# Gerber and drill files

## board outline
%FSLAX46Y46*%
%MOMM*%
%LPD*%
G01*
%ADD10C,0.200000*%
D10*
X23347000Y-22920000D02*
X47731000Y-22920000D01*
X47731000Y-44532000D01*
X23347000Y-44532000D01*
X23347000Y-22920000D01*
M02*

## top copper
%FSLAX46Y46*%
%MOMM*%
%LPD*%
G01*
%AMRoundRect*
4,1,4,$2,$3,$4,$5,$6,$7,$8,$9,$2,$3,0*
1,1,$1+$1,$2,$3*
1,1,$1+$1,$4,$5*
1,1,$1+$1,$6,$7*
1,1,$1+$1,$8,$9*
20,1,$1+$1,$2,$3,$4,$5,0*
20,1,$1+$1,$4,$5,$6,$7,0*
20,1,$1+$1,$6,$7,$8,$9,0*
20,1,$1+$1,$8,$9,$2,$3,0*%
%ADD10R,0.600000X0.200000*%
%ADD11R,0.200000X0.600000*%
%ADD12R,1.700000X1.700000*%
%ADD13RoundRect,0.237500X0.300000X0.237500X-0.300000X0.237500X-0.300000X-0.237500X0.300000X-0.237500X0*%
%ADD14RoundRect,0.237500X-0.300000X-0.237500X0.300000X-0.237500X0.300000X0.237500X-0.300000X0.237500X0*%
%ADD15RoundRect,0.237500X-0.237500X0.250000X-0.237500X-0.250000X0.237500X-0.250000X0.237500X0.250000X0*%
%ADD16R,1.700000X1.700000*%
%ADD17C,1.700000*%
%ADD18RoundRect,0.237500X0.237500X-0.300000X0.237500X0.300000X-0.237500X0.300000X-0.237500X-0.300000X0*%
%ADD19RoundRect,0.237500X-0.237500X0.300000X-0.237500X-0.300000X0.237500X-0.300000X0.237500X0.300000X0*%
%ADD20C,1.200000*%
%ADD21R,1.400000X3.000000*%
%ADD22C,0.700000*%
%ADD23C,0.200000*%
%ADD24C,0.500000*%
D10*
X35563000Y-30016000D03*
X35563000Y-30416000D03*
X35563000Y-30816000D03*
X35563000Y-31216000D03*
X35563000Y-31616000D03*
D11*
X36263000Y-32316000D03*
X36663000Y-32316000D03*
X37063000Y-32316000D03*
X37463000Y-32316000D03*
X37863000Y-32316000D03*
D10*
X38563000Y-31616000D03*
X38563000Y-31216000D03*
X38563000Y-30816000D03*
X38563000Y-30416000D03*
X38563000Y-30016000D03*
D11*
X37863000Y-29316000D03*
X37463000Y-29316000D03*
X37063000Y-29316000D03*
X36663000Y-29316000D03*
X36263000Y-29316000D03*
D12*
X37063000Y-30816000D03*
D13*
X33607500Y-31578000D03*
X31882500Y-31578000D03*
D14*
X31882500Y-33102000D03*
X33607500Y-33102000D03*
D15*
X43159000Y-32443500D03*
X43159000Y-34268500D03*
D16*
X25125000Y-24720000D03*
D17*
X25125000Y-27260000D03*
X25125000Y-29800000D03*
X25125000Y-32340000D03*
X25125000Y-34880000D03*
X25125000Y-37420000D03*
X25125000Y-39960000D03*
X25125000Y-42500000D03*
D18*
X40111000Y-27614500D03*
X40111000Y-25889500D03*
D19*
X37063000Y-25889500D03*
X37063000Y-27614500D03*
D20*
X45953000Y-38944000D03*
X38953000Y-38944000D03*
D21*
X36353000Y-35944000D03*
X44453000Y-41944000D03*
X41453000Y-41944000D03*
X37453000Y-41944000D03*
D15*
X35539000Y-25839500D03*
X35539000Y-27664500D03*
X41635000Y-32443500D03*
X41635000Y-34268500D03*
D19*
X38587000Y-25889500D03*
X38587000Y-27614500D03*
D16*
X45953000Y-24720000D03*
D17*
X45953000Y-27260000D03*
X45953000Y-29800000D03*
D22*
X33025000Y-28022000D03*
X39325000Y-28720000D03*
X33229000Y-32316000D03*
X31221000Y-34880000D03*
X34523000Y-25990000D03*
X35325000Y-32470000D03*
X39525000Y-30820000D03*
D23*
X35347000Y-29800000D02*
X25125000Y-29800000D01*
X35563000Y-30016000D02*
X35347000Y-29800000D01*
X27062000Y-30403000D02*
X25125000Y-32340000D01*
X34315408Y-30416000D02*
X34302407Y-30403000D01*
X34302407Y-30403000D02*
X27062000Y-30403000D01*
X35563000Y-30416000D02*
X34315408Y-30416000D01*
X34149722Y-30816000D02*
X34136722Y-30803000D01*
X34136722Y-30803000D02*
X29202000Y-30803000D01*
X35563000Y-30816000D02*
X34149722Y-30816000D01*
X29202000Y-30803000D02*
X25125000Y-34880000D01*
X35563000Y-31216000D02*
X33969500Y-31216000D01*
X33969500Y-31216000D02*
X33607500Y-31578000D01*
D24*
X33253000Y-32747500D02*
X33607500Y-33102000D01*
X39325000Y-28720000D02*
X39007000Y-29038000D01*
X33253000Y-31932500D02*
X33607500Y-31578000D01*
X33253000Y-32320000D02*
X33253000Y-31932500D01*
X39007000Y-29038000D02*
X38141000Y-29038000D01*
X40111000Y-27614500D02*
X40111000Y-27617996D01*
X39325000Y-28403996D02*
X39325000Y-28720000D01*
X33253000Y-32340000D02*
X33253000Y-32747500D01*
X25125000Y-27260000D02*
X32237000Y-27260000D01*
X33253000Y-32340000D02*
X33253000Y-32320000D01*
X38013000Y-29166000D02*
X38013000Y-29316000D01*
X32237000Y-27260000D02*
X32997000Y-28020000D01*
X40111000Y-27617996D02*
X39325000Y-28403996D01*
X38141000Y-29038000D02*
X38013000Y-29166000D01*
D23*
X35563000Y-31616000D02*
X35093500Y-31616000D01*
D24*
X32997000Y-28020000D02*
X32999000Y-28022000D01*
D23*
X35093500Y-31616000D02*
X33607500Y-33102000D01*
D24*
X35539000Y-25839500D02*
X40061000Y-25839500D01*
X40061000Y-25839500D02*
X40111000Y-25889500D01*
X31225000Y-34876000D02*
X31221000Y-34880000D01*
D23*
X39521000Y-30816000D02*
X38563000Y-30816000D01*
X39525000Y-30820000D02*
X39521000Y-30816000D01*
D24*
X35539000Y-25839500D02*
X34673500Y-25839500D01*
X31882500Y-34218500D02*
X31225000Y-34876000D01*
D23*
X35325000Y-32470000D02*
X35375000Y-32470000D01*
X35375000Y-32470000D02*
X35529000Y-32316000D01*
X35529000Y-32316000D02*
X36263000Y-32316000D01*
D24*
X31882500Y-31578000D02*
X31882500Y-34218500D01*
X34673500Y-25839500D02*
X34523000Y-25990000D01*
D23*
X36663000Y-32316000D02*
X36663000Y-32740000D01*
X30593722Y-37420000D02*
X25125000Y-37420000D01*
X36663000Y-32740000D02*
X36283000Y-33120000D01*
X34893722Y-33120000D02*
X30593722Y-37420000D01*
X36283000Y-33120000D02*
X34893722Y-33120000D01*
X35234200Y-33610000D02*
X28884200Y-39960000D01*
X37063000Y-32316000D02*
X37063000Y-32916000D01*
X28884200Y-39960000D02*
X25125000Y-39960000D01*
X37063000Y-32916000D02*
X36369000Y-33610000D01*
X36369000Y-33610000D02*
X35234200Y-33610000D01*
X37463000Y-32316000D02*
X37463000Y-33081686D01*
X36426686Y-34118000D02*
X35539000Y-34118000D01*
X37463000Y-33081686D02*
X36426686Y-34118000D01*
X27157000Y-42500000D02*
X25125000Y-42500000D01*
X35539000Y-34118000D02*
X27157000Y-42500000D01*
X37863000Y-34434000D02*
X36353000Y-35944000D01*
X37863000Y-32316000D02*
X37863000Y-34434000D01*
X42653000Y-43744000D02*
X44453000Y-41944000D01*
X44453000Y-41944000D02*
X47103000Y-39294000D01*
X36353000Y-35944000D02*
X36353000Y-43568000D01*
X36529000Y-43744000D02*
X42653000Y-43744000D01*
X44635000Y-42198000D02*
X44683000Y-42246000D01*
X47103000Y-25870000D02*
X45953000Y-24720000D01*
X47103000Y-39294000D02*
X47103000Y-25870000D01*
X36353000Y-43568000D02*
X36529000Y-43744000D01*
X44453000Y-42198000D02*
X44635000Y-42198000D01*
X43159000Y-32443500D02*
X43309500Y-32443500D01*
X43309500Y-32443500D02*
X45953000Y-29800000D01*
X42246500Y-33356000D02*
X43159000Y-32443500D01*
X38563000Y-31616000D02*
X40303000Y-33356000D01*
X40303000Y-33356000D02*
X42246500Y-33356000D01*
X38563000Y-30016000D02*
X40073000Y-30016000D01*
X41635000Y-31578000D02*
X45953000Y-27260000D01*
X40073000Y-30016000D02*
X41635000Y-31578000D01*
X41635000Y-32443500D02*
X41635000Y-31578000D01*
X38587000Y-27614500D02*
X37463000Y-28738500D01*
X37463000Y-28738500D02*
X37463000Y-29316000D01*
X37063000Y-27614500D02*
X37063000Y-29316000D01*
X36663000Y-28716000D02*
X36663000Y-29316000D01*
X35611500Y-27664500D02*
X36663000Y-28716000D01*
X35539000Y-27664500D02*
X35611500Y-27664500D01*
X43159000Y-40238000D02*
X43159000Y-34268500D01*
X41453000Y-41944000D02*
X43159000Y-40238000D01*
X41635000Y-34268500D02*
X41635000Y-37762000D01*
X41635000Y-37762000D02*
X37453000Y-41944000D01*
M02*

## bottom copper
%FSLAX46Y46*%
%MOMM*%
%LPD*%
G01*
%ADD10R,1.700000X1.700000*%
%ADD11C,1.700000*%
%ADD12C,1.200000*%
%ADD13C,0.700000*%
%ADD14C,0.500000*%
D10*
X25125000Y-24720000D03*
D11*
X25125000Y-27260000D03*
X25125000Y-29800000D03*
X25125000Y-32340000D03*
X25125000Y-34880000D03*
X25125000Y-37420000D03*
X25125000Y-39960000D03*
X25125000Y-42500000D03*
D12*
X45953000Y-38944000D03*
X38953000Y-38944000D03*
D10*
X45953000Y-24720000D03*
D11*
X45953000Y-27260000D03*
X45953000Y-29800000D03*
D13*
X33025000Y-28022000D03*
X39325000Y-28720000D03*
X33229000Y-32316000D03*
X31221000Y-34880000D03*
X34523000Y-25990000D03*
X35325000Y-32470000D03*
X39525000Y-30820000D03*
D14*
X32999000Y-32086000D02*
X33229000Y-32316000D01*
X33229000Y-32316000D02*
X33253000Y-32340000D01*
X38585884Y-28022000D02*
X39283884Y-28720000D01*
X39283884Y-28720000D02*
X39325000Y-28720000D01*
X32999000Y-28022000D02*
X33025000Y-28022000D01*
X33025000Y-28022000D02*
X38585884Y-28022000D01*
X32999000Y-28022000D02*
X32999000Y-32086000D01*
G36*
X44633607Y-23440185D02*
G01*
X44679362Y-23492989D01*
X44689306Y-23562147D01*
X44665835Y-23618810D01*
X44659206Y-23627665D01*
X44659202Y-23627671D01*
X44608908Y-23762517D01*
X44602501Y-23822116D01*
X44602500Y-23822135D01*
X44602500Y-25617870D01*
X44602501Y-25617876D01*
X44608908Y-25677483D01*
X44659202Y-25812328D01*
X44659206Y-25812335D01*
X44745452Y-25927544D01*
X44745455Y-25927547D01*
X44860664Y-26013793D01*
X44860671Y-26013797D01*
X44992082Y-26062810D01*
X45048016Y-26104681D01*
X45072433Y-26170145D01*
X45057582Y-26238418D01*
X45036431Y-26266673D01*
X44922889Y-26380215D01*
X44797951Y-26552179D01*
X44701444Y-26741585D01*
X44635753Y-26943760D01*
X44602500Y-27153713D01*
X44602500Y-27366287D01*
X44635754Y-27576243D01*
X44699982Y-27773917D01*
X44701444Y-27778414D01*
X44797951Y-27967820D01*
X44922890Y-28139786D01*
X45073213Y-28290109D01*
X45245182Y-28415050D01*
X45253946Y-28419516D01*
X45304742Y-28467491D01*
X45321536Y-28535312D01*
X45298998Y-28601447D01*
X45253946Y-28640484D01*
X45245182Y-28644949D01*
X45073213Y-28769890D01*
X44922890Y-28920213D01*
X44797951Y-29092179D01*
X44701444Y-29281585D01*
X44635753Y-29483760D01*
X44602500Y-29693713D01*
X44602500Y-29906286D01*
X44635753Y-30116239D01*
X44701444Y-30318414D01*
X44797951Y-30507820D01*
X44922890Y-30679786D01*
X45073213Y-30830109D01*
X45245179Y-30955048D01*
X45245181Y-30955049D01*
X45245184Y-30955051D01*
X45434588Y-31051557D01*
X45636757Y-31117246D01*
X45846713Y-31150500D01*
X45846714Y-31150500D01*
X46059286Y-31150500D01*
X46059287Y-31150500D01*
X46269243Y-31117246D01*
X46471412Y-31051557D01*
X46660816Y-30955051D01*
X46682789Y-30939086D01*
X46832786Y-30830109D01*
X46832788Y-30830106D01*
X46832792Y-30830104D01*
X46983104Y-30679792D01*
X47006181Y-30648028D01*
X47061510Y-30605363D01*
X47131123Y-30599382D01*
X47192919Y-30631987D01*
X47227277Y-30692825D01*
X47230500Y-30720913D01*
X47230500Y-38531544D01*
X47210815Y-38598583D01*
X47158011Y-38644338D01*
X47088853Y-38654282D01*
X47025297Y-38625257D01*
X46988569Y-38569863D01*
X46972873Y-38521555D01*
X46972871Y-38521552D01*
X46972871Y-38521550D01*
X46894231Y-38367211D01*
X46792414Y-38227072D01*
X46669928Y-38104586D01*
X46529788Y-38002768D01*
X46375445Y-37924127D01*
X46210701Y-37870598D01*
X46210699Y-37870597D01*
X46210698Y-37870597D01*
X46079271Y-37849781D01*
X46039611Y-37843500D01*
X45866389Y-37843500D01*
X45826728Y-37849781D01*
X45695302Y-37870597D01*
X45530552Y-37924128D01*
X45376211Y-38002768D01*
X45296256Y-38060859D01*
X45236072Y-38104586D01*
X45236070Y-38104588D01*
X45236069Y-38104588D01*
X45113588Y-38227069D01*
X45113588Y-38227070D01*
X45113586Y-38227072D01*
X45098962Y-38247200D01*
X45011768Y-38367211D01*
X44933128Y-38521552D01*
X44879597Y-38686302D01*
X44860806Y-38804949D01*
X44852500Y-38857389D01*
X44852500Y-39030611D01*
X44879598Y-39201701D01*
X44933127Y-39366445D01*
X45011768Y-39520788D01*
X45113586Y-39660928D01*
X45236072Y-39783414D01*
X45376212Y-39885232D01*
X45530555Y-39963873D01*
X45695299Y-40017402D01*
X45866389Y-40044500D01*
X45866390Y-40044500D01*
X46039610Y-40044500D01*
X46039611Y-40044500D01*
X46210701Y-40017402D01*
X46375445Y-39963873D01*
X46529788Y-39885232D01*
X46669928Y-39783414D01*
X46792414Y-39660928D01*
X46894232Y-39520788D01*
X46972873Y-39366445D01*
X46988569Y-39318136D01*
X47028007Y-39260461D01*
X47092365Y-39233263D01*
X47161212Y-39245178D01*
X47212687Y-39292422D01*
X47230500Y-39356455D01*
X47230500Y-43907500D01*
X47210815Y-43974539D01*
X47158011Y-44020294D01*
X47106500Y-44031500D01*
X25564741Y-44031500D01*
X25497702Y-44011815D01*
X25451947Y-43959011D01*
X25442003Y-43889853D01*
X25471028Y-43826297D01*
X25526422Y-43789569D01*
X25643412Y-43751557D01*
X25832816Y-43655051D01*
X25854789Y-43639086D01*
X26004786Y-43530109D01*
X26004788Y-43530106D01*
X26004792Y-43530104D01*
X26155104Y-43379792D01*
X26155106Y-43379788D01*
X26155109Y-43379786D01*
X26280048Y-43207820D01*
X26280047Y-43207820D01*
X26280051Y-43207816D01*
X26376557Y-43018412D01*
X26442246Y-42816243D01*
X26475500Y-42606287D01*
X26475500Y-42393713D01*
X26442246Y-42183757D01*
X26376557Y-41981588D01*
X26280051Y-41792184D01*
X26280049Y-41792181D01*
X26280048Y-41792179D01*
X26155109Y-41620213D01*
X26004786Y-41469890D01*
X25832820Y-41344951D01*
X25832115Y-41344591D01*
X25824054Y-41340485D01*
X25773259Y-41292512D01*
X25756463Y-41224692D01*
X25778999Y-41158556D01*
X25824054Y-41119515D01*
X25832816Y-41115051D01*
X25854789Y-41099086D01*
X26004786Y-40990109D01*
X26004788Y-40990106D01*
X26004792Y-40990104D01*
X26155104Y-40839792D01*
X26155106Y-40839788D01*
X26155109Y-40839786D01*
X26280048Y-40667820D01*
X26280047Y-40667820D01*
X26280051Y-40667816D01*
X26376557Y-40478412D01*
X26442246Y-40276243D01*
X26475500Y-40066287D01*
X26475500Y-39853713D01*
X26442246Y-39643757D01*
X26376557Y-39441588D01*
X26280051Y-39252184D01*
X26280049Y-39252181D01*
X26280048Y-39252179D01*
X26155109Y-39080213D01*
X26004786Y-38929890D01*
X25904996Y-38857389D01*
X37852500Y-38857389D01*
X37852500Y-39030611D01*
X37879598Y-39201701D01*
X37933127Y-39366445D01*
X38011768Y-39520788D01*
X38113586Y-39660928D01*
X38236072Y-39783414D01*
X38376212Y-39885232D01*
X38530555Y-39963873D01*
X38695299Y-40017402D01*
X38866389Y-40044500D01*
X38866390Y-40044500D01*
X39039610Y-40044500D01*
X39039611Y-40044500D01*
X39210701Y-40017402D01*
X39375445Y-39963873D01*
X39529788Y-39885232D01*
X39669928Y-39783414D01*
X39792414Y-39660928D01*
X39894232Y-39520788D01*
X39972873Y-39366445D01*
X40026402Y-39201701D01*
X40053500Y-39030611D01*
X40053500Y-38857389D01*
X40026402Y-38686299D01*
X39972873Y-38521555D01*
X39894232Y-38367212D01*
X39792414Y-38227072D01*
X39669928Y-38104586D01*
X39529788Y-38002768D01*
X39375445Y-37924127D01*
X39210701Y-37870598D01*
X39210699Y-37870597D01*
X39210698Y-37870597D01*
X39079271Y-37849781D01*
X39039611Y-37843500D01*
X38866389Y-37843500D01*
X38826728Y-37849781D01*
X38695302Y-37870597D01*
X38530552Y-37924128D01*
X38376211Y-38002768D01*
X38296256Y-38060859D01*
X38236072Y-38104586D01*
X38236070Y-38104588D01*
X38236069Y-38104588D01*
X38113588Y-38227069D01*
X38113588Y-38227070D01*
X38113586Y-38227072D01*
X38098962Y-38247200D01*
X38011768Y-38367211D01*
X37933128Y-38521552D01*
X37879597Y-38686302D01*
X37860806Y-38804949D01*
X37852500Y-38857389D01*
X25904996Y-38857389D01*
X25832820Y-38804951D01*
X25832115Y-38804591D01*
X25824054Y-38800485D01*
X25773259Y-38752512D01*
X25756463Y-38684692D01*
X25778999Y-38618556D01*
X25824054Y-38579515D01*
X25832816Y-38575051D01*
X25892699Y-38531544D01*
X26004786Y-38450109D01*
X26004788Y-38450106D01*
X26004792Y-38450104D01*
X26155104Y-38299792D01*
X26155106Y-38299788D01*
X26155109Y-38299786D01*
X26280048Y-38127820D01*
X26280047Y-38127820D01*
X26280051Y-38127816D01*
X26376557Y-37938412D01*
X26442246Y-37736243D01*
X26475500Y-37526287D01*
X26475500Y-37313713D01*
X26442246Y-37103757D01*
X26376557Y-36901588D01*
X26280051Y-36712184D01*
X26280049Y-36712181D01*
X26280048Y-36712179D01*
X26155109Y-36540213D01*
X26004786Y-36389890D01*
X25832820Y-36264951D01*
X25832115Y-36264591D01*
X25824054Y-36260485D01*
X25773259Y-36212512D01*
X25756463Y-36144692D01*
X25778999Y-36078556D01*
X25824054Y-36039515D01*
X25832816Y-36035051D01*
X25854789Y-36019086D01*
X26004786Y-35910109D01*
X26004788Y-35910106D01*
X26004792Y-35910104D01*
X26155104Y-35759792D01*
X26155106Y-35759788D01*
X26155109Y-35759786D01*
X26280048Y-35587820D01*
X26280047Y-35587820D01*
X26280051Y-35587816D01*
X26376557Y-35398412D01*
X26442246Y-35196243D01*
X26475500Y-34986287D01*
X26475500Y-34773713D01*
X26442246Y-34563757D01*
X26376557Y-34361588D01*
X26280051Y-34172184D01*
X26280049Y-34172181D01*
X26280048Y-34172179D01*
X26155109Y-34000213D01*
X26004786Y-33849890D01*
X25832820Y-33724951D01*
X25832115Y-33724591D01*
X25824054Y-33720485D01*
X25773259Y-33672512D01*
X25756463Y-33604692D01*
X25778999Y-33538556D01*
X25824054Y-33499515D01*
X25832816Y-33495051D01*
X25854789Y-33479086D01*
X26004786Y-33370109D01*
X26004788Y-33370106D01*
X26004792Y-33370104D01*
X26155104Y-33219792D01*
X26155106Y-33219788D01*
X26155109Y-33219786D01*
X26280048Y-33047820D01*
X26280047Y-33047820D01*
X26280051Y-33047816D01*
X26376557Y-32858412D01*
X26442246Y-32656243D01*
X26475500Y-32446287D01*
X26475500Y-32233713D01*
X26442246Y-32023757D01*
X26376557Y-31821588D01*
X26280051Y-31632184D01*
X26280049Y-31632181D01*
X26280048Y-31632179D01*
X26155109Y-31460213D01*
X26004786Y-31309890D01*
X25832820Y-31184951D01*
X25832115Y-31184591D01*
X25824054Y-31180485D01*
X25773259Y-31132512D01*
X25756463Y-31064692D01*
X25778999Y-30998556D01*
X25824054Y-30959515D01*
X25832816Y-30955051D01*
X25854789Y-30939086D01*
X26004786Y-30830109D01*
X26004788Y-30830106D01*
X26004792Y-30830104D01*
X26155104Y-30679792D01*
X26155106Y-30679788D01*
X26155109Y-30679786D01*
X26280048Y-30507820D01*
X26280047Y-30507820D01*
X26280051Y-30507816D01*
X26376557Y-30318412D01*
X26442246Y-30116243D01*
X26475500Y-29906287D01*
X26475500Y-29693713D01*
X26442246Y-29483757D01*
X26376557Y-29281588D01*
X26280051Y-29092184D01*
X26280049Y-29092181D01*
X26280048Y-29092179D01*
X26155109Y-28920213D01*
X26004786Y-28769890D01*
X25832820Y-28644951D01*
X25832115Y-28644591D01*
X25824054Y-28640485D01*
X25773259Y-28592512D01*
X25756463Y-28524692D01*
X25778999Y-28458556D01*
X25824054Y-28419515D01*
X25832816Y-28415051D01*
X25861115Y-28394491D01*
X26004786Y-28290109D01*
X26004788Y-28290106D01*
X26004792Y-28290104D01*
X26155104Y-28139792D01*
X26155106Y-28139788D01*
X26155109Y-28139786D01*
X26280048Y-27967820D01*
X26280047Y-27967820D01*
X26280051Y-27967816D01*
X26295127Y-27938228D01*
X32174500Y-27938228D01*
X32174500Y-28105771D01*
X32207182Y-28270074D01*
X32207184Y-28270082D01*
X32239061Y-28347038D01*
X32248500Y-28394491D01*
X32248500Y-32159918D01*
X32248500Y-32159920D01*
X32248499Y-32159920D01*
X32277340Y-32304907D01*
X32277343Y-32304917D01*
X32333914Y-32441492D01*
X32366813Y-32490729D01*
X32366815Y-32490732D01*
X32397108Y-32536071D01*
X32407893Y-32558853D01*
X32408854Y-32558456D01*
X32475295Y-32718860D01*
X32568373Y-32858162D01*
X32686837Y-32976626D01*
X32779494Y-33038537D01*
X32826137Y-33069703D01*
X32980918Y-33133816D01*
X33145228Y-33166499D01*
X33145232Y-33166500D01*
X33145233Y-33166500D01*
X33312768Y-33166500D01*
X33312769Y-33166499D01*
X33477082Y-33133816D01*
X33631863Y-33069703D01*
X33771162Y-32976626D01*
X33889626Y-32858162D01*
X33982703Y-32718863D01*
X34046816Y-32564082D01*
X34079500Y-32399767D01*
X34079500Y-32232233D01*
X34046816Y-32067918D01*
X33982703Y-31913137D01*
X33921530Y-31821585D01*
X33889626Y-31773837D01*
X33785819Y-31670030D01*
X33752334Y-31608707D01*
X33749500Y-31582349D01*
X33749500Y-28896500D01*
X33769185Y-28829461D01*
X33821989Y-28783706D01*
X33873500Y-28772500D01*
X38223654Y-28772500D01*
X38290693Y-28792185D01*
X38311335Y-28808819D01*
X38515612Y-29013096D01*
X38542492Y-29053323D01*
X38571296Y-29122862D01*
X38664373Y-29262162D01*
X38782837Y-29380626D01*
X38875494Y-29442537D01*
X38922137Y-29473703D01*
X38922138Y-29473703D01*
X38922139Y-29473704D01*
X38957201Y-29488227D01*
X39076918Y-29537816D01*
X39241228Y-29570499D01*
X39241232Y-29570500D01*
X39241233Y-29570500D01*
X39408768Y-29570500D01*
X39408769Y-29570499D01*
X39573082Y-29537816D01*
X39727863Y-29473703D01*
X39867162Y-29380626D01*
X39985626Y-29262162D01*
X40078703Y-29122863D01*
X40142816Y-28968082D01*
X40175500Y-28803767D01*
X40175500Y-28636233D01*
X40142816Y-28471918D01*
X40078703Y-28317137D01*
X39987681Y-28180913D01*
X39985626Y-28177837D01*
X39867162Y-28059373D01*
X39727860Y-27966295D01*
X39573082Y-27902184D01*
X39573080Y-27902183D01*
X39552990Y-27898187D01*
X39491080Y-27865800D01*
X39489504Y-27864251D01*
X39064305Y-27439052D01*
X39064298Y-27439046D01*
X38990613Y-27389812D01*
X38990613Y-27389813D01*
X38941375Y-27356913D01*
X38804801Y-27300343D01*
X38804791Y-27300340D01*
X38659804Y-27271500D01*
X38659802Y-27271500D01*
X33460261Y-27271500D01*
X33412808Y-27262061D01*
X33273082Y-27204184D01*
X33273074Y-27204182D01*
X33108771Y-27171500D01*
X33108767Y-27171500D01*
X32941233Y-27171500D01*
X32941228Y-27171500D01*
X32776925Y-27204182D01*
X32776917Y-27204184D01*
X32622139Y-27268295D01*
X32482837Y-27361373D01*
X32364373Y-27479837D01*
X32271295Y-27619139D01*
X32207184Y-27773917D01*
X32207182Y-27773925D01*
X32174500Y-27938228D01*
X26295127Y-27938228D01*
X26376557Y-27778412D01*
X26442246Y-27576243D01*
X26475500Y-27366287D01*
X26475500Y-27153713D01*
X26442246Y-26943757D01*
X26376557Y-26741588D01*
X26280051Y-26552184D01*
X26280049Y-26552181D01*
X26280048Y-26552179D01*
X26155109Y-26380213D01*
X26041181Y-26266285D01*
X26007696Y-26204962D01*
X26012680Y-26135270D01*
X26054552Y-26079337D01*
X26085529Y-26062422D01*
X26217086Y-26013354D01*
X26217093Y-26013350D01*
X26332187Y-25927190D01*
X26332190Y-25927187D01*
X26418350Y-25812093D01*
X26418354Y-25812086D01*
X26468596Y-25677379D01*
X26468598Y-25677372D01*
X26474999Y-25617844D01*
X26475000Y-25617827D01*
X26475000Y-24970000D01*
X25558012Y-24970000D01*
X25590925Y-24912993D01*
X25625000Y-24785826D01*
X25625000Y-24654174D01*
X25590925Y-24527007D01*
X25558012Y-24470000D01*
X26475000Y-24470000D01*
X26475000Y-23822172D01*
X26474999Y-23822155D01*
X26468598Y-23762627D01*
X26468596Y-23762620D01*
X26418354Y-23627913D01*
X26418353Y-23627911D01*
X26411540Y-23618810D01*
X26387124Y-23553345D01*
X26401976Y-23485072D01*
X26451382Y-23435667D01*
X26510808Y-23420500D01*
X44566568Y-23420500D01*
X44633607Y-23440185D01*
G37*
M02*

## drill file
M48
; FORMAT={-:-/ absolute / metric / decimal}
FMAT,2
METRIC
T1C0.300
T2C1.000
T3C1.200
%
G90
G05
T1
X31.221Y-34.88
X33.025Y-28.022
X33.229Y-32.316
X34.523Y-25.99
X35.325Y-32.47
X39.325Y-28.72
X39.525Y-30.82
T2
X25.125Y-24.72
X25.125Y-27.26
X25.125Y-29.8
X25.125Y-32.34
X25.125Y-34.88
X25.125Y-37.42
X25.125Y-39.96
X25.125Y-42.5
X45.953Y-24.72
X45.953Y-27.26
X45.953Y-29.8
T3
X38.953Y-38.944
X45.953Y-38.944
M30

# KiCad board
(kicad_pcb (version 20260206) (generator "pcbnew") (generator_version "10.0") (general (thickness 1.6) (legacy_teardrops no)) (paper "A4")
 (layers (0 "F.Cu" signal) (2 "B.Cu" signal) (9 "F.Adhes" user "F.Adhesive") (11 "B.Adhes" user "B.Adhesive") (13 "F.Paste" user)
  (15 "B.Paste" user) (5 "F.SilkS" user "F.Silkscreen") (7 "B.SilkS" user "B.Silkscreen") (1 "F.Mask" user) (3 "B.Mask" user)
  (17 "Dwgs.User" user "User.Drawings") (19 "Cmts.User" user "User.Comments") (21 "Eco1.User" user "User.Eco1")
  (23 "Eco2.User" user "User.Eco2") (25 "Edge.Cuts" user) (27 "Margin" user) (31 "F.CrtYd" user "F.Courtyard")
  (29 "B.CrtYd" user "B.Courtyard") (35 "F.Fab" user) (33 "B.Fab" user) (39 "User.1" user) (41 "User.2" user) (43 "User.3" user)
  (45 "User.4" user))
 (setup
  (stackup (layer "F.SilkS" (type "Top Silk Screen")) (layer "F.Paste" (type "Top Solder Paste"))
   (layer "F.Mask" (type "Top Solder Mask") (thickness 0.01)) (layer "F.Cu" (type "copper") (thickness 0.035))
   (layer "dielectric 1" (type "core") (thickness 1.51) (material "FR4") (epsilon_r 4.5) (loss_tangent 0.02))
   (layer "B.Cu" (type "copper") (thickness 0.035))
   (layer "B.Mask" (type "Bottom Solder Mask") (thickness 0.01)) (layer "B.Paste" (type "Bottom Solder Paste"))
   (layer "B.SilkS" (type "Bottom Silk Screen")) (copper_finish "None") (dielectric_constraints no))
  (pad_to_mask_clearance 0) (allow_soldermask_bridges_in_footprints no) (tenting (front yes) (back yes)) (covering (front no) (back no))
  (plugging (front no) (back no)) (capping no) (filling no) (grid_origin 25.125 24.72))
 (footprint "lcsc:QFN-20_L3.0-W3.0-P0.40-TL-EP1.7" (layer "F.Cu") (at 37.063 30.816)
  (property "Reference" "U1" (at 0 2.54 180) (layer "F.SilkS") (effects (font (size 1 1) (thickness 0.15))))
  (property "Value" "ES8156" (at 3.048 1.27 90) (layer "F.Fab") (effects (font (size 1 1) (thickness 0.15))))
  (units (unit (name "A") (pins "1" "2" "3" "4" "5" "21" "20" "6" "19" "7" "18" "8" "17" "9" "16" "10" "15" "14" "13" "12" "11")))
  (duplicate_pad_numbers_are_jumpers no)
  (pad "1" smd rect (at -1.5 -0.8) (size 0.6 0.2) (layers "F.Cu" "F.Mask" "F.Paste") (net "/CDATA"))
  (pad "2" smd rect (at -1.5 -0.4) (size 0.6 0.2) (layers "F.Cu" "F.Mask" "F.Paste") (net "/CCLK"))
  (pad "3" smd rect (at -1.5 0) (size 0.6 0.2) (layers "F.Cu" "F.Mask" "F.Paste") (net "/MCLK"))
  (pad "4" smd rect (at -1.5 0.4) (size 0.6 0.2) (layers "F.Cu" "F.Mask" "F.Paste") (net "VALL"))
  (pad "5" smd rect (at -1.5 0.8) (size 0.6 0.2) (layers "F.Cu" "F.Mask" "F.Paste") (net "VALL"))
  (pad "6" smd rect (at -0.8 1.5) (size 0.2 0.6) (layers "F.Cu" "F.Mask" "F.Paste") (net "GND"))
  (pad "7" smd rect (at -0.4 1.5) (size 0.2 0.6) (layers "F.Cu" "F.Mask" "F.Paste") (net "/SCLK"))
  (pad "8" smd rect (at 0 1.5) (size 0.2 0.6) (layers "F.Cu" "F.Mask" "F.Paste") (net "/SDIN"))
  (pad "9" smd rect (at 0.4 1.5) (size 0.2 0.6) (layers "F.Cu" "F.Mask" "F.Paste") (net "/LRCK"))
  (pad "10" smd rect (at 0.8 1.5) (size 0.2 0.6) (layers "F.Cu" "F.Mask" "F.Paste") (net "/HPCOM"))
  (pad "11" smd rect (at 1.5 0.8) (size 0.6 0.2) (layers "F.Cu" "F.Mask" "F.Paste") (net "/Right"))
  (pad "12" smd rect (at 1.5 0.4) (size 0.6 0.2) (layers "F.Cu" "F.Mask" "F.Paste") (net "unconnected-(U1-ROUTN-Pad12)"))
  (pad "13" smd rect (at 1.5 0) (size 0.6 0.2) (layers "F.Cu" "F.Mask" "F.Paste") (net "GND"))
  (pad "14" smd rect (at 1.5 -0.4) (size 0.6 0.2) (layers "F.Cu" "F.Mask" "F.Paste") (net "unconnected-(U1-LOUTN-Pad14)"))
  (pad "15" smd rect (at 1.5 -0.8) (size 0.6 0.2) (layers "F.Cu" "F.Mask" "F.Paste") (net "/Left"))
  (pad "16" smd rect (at 0.8 -1.5) (size 0.2 0.6) (layers "F.Cu" "F.Mask" "F.Paste") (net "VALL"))
  (pad "17" smd rect (at 0.4 -1.5) (size 0.2 0.6) (layers "F.Cu" "F.Mask" "F.Paste") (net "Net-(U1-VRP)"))
  (pad "18" smd rect (at 0 -1.5) (size 0.2 0.6) (layers "F.Cu" "F.Mask" "F.Paste") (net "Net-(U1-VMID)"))
  (pad "19" smd rect (at -0.4 -1.5) (size 0.2 0.6) (layers "F.Cu" "F.Mask" "F.Paste") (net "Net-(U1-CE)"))
  (pad "20" smd rect (at -0.8 -1.5) (size 0.2 0.6) (layers "F.Cu" "F.Mask" "F.Paste") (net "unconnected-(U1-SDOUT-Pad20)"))
  (pad "21" smd rect (at 0 0 180) (size 1.7 1.7) (layers "F.Cu" "F.Mask" "F.Paste") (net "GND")))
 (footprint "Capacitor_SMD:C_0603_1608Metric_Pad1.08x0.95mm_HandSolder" (layer "F.Cu") (at 32.745 31.578 180)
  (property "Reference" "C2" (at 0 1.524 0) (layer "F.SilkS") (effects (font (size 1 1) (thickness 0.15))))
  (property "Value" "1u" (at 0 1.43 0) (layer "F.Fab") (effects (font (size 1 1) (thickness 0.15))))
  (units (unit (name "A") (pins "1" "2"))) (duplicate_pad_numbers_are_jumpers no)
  (pad "1" smd roundrect (at -0.8625 0 180) (size 1.075 0.95) (layers "F.Cu" "F.Mask" "F.Paste") (roundrect_rratio 0.25) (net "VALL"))
  (pad "2" smd roundrect (at 0.8625 0 180) (size 1.075 0.95) (layers "F.Cu" "F.Mask" "F.Paste") (roundrect_rratio 0.25) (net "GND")))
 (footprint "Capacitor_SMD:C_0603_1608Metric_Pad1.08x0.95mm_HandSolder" (layer "F.Cu") (at 32.745 33.102)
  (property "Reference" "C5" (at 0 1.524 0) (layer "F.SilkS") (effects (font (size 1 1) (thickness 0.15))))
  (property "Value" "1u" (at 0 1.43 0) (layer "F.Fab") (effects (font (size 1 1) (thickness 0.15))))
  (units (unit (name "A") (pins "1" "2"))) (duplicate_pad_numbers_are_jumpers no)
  (pad "1" smd roundrect (at -0.8625 0) (size 1.075 0.95) (layers "F.Cu" "F.Mask" "F.Paste") (roundrect_rratio 0.25) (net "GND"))
  (pad "2" smd roundrect (at 0.8625 0) (size 1.075 0.95) (layers "F.Cu" "F.Mask" "F.Paste") (roundrect_rratio 0.25) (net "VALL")))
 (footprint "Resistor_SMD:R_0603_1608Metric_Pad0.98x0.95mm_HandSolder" (layer "F.Cu") (at 43.159 33.356 -90)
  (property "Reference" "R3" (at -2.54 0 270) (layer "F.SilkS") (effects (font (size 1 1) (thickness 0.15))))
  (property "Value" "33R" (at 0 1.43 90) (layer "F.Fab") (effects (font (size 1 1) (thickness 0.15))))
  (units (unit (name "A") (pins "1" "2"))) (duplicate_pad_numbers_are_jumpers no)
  (pad "1" smd roundrect (at -0.9125 0 270) (size 0.975 0.95) (layers "F.Cu" "F.Mask" "F.Paste") (roundrect_rratio 0.25) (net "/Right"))
  (pad "2" smd roundrect (at 0.9125 0 270) (size 0.975 0.95) (layers "F.Cu" "F.Mask" "F.Paste") (roundrect_rratio 0.25) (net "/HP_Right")))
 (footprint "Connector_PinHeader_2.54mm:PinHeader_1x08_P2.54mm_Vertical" (layer "F.Cu") (at 25.125 24.72)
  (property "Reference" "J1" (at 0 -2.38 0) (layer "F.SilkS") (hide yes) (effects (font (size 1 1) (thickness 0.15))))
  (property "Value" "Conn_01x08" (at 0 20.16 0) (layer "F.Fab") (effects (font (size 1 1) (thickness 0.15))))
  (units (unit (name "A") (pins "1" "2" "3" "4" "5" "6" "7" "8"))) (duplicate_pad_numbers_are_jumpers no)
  (pad "1" thru_hole rect (at 0 0) (size 1.7 1.7) (drill 1) (layers "*.Cu" "*.Mask") (remove_unused_layers no) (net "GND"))
  (pad "2" thru_hole circle (at 0 2.54) (size 1.7 1.7) (drill 1) (layers "*.Cu" "*.Mask") (remove_unused_layers no) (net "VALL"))
  (pad "3" thru_hole circle (at 0 5.08) (size 1.7 1.7) (drill 1) (layers "*.Cu" "*.Mask") (remove_unused_layers no) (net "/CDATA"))
  (pad "4" thru_hole circle (at 0 7.62) (size 1.7 1.7) (drill 1) (layers "*.Cu" "*.Mask") (remove_unused_layers no) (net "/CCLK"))
  (pad "5" thru_hole circle (at 0 10.16) (size 1.7 1.7) (drill 1) (layers "*.Cu" "*.Mask") (remove_unused_layers no) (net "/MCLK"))
  (pad "6" thru_hole circle (at 0 12.7) (size 1.7 1.7) (drill 1) (layers "*.Cu" "*.Mask") (remove_unused_layers no) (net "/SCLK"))
  (pad "7" thru_hole circle (at 0 15.24) (size 1.7 1.7) (drill 1) (layers "*.Cu" "*.Mask") (remove_unused_layers no) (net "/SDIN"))
  (pad "8" thru_hole circle (at 0 17.78) (size 1.7 1.7) (drill 1) (layers "*.Cu" "*.Mask") (remove_unused_layers no) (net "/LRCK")))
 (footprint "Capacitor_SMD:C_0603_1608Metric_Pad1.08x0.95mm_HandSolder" (layer "F.Cu") (at 40.111 26.752 90)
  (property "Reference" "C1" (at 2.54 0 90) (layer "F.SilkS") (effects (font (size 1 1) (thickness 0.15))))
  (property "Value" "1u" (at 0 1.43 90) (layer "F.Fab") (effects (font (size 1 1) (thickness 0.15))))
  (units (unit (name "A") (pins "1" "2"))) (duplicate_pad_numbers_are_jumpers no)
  (pad "1" smd roundrect (at -0.8625 0 90) (size 1.075 0.95) (layers "F.Cu" "F.Mask" "F.Paste") (roundrect_rratio 0.25) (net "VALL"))
  (pad "2" smd roundrect (at 0.8625 0 90) (size 1.075 0.95) (layers "F.Cu" "F.Mask" "F.Paste") (roundrect_rratio 0.25) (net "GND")))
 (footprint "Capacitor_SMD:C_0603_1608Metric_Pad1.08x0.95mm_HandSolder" (layer "F.Cu") (at 37.063 26.752 -90)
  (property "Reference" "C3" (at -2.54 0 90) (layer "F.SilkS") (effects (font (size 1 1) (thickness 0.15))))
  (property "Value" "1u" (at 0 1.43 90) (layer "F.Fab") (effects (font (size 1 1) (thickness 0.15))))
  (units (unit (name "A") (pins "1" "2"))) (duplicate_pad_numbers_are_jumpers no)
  (pad "1" smd roundrect (at -0.8625 0 270) (size 1.075 0.95) (layers "F.Cu" "F.Mask" "F.Paste") (roundrect_rratio 0.25) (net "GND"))
  (pad "2" smd roundrect (at 0.8625 0 270) (size 1.075 0.95) (layers "F.Cu" "F.Mask" "F.Paste") (roundrect_rratio 0.25)
   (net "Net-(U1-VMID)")))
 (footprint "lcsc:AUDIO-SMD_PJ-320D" (layer "F.Cu") (at 40.403 38.944 -90)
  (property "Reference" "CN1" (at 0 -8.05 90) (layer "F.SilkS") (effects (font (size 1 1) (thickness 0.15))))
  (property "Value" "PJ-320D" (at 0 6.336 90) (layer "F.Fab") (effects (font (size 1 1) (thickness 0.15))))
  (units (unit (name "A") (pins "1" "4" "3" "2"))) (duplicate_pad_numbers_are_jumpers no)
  (pad "" thru_hole circle (at 0 -5.55 270) (size 1.2 1.2) (drill 1.2) (layers "*.Cu" "*.Mask") (remove_unused_layers no))
  (pad "" thru_hole circle (at 0 1.45 270) (size 1.2 1.2) (drill 1.2) (layers "*.Cu" "*.Mask") (remove_unused_layers no))
  (pad "1" smd rect (at -3 4.05 270) (size 3 1.4) (layers "F.Cu" "F.Mask" "F.Paste") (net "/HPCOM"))
  (pad "2" smd rect (at 3 -4.05 270) (size 3 1.4) (layers "F.Cu" "F.Mask" "F.Paste") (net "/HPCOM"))
  (pad "3" smd rect (at 3 -1.05 270) (size 3 1.4) (layers "F.Cu" "F.Mask" "F.Paste") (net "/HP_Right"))
  (pad "4" smd rect (at 3 2.95 270) (size 3 1.4) (layers "F.Cu" "F.Mask" "F.Paste") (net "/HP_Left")))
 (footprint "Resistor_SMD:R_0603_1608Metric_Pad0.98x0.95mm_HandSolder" (layer "F.Cu") (at 35.539 26.752 -90)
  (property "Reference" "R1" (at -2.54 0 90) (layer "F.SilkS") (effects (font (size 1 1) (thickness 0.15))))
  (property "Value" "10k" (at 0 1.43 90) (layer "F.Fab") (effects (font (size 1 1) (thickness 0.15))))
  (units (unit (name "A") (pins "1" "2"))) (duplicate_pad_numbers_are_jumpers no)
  (pad "1" smd roundrect (at -0.9125 0 270) (size 0.975 0.95) (layers "F.Cu" "F.Mask" "F.Paste") (roundrect_rratio 0.25) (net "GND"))
  (pad "2" smd roundrect (at 0.9125 0 270) (size 0.975 0.95) (layers "F.Cu" "F.Mask" "F.Paste") (roundrect_rratio 0.25) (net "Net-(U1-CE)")))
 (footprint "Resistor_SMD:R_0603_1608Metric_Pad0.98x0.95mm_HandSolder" (layer "F.Cu") (at 41.635 33.356 -90)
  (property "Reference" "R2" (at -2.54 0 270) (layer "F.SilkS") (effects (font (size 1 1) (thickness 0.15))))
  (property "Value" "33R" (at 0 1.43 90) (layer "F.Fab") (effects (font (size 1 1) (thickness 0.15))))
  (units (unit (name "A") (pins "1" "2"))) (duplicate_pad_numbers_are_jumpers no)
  (pad "1" smd roundrect (at -0.9125 0 270) (size 0.975 0.95) (layers "F.Cu" "F.Mask" "F.Paste") (roundrect_rratio 0.25) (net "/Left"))
  (pad "2" smd roundrect (at 0.9125 0 270) (size 0.975 0.95) (layers "F.Cu" "F.Mask" "F.Paste") (roundrect_rratio 0.25) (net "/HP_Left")))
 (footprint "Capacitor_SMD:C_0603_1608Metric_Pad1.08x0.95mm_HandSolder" (layer "F.Cu") (at 38.587 26.752 -90)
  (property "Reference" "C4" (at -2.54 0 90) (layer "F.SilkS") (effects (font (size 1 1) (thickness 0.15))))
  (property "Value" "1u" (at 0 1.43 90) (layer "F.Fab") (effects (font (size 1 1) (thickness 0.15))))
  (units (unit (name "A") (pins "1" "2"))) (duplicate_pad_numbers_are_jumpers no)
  (pad "1" smd roundrect (at -0.8625 0 270) (size 1.075 0.95) (layers "F.Cu" "F.Mask" "F.Paste") (roundrect_rratio 0.25) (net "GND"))
  (pad "2" smd roundrect (at 0.8625 0 270) (size 1.075 0.95) (layers "F.Cu" "F.Mask" "F.Paste") (roundrect_rratio 0.25) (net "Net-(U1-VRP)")))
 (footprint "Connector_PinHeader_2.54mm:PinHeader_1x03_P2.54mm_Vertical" (layer "F.Cu") (at 45.953 24.72)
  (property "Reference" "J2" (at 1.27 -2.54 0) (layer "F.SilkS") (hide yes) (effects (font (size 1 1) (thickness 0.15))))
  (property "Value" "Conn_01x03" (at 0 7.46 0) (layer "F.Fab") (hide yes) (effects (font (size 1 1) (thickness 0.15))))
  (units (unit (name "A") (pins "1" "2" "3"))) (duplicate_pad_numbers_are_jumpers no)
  (pad "1" thru_hole rect (at 0 0) (size 1.7 1.7) (drill 1) (layers "*.Cu" "*.Mask") (remove_unused_layers no) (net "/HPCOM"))
  (pad "2" thru_hole circle (at 0 2.54) (size 1.7 1.7) (drill 1) (layers "*.Cu" "*.Mask") (remove_unused_layers no) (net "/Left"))
  (pad "3" thru_hole circle (at 0 5.08) (size 1.7 1.7) (drill 1) (layers "*.Cu" "*.Mask") (remove_unused_layers no) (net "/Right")))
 (gr_rect (start 23.347 22.92) (end 47.731 44.532) (stroke (width 0.2) (type solid)) (fill no) (layer "Edge.Cuts"))
 (segment (start 35.347 29.8) (end 25.125 29.8) (width 0.2) (layer "F.Cu") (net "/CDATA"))
 (segment (start 35.563 30.016) (end 35.347 29.8) (width 0.2) (layer "F.Cu") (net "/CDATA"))
 (segment (start 27.062 30.403) (end 25.125 32.34) (width 0.2) (layer "F.Cu") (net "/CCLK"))
 (segment (start 34.315408 30.416) (end 34.302407 30.403) (width 0.2) (layer "F.Cu") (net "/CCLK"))
 (segment (start 34.302407 30.403) (end 27.062 30.403) (width 0.2) (layer "F.Cu") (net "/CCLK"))
 (segment (start 35.563 30.416) (end 34.315408 30.416) (width 0.2) (layer "F.Cu") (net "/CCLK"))
 (segment (start 34.149722 30.816) (end 34.136722 30.803) (width 0.2) (layer "F.Cu") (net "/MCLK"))
 (segment (start 34.136722 30.803) (end 29.202 30.803) (width 0.2) (layer "F.Cu") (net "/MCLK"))
 (segment (start 35.563 30.816) (end 34.149722 30.816) (width 0.2) (layer "F.Cu") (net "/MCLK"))
 (segment (start 29.202 30.803) (end 25.125 34.88) (width 0.2) (layer "F.Cu") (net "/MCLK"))
 (segment (start 35.563 31.216) (end 33.9695 31.216) (width 0.2) (layer "F.Cu") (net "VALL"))
 (segment (start 33.9695 31.216) (end 33.6075 31.578) (width 0.2) (layer "F.Cu") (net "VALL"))
 (segment (start 33.253 32.7475) (end 33.6075 33.102) (width 0.5) (layer "F.Cu") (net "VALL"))
 (segment (start 39.325 28.72) (end 39.007 29.038) (width 0.5) (layer "F.Cu") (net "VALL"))
 (segment (start 33.253 31.9325) (end 33.6075 31.578) (width 0.5) (layer "F.Cu") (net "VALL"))
 (segment (start 33.253 32.32) (end 33.253 31.9325) (width 0.5) (layer "F.Cu") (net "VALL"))
 (segment (start 39.007 29.038) (end 38.141 29.038) (width 0.5) (layer "F.Cu") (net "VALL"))
 (segment (start 40.111 27.6145) (end 40.111 27.617996) (width 0.5) (layer "F.Cu") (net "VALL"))
 (segment (start 39.325 28.403996) (end 39.325 28.72) (width 0.5) (layer "F.Cu") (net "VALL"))
 (segment (start 33.253 32.34) (end 33.253 32.7475) (width 0.5) (layer "F.Cu") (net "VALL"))
 (segment (start 25.125 27.26) (end 32.237 27.26) (width 0.5) (layer "F.Cu") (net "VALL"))
 (segment (start 33.253 32.34) (end 33.253 32.32) (width 0.5) (layer "F.Cu") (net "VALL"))
 (segment (start 38.013 29.166) (end 38.013 29.316) (width 0.5) (layer "F.Cu") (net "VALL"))
 (segment (start 32.237 27.26) (end 32.997 28.02) (width 0.5) (layer "F.Cu") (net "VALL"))
 (segment (start 40.111 27.617996) (end 39.325 28.403996) (width 0.5) (layer "F.Cu") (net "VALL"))
 (segment (start 38.141 29.038) (end 38.013 29.166) (width 0.5) (layer "F.Cu") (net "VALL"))
 (segment (start 35.563 31.616) (end 35.0935 31.616) (width 0.2) (layer "F.Cu") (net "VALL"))
 (segment (start 32.997 28.02) (end 32.999 28.022) (width 0.5) (layer "F.Cu") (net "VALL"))
 (segment (start 35.0935 31.616) (end 33.6075 33.102) (width 0.2) (layer "F.Cu") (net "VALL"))
 (via (at 33.025 28.022) (size 0.7) (drill 0.3) (layers "F.Cu" "B.Cu") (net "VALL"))
 (via (at 39.325 28.72) (size 0.7) (drill 0.3) (layers "F.Cu" "B.Cu") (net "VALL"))
 (via (at 33.229 32.316) (size 0.7) (drill 0.3) (layers "F.Cu" "B.Cu") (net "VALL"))
 (segment (start 32.999 32.086) (end 33.229 32.316) (width 0.5) (layer "B.Cu") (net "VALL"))
 (segment (start 33.229 32.316) (end 33.253 32.34) (width 0.5) (layer "B.Cu") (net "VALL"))
 (segment (start 38.585884 28.022) (end 39.283884 28.72) (width 0.5) (layer "B.Cu") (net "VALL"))
 (segment (start 39.283884 28.72) (end 39.325 28.72) (width 0.5) (layer "B.Cu") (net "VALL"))
 (segment (start 32.999 28.022) (end 33.025 28.022) (width 0.5) (layer "B.Cu") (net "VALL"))
 (segment (start 33.025 28.022) (end 38.585884 28.022) (width 0.5) (layer "B.Cu") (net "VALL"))
 (segment (start 32.999 28.022) (end 32.999 32.086) (width 0.5) (layer "B.Cu") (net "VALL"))
 (segment (start 35.539 25.8395) (end 40.061 25.8395) (width 0.5) (layer "F.Cu") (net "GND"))
 (segment (start 40.061 25.8395) (end 40.111 25.8895) (width 0.5) (layer "F.Cu") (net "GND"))
 (segment (start 31.225 34.876) (end 31.221 34.88) (width 0.5) (layer "F.Cu") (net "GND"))
 (segment (start 39.521 30.816) (end 38.563 30.816) (width 0.2) (layer "F.Cu") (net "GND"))
 (segment (start 39.525 30.82) (end 39.521 30.816) (width 0.2) (layer "F.Cu") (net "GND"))
 (segment (start 35.539 25.8395) (end 34.6735 25.8395) (width 0.5) (layer "F.Cu") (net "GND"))
 (segment (start 31.8825 34.2185) (end 31.225 34.876) (width 0.5) (layer "F.Cu") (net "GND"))
 (segment (start 35.325 32.47) (end 35.375 32.47) (width 0.2) (layer "F.Cu") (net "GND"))
 (segment (start 35.375 32.47) (end 35.529 32.316) (width 0.2) (layer "F.Cu") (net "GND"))
 (segment (start 35.529 32.316) (end 36.263 32.316) (width 0.2) (layer "F.Cu") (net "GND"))
 (segment (start 31.8825 31.578) (end 31.8825 34.2185) (width 0.5) (layer "F.Cu") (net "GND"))
 (segment (start 34.6735 25.8395) (end 34.523 25.99) (width 0.5) (layer "F.Cu") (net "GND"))
 (via (at 31.221 34.88) (size 0.7) (drill 0.3) (layers "F.Cu" "B.Cu") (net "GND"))
 (via (at 34.523 25.99) (size 0.7) (drill 0.3) (layers "F.Cu" "B.Cu") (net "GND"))
 (via (at 35.325 32.47) (size 0.7) (drill 0.3) (layers "F.Cu" "B.Cu") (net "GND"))
 (via (at 39.525 30.82) (size 0.7) (drill 0.3) (layers "F.Cu" "B.Cu") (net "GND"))
 (segment (start 36.663 32.316) (end 36.663 32.74) (width 0.2) (layer "F.Cu") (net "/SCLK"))
 (segment (start 30.593722 37.42) (end 25.125 37.42) (width 0.2) (layer "F.Cu") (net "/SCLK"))
 (segment (start 36.663 32.74) (end 36.283 33.12) (width 0.2) (layer "F.Cu") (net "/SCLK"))
 (segment (start 34.893722 33.12) (end 30.593722 37.42) (width 0.2) (layer "F.Cu") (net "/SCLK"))
 (segment (start 36.283 33.12) (end 34.893722 33.12) (width 0.2) (layer "F.Cu") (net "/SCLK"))
 (segment (start 35.2342 33.61) (end 28.8842 39.96) (width 0.2) (layer "F.Cu") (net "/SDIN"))
 (segment (start 37.063 32.316) (end 37.063 32.916) (width 0.2) (layer "F.Cu") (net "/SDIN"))
 (segment (start 28.8842 39.96) (end 25.125 39.96) (width 0.2) (layer "F.Cu") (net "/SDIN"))
 (segment (start 37.063 32.916) (end 36.369 33.61) (width 0.2) (layer "F.Cu") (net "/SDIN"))
 (segment (start 36.369 33.61) (end 35.2342 33.61) (width 0.2) (layer "F.Cu") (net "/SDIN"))
 (segment (start 37.463 32.316) (end 37.463 33.081686) (width 0.2) (layer "F.Cu") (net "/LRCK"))
 (segment (start 36.426686 34.118) (end 35.539 34.118) (width 0.2) (layer "F.Cu") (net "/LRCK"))
 (segment (start 37.463 33.081686) (end 36.426686 34.118) (width 0.2) (layer "F.Cu") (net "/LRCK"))
 (segment (start 27.157 42.5) (end 25.125 42.5) (width 0.2) (layer "F.Cu") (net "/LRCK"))
 (segment (start 35.539 34.118) (end 27.157 42.5) (width 0.2) (layer "F.Cu") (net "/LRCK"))
 (segment (start 37.863 34.434) (end 36.353 35.944) (width 0.2) (layer "F.Cu") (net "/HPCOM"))
 (segment (start 37.863 32.316) (end 37.863 34.434) (width 0.2) (layer "F.Cu") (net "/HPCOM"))
 (segment (start 42.653 43.744) (end 44.453 41.944) (width 0.2) (layer "F.Cu") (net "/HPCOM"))
 (segment (start 44.453 41.944) (end 47.103 39.294) (width 0.2) (layer "F.Cu") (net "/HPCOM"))
 (segment (start 36.353 35.944) (end 36.353 43.568) (width 0.2) (layer "F.Cu") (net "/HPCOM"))
 (segment (start 36.529 43.744) (end 42.653 43.744) (width 0.2) (layer "F.Cu") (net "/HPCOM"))
 (segment (start 44.635 42.198) (end 44.683 42.246) (width 0.2) (layer "F.Cu") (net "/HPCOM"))
 (segment (start 47.103 25.87) (end 45.953 24.72) (width 0.2) (layer "F.Cu") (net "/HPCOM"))
 (segment (start 47.103 39.294) (end 47.103 25.87) (width 0.2) (layer "F.Cu") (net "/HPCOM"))
 (segment (start 36.353 43.568) (end 36.529 43.744) (width 0.2) (layer "F.Cu") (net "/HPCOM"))
 (segment (start 44.453 42.198) (end 44.635 42.198) (width 0.2) (layer "F.Cu") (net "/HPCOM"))
 (segment (start 43.159 32.4435) (end 43.3095 32.4435) (width 0.2) (layer "F.Cu") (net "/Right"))
 (segment (start 43.3095 32.4435) (end 45.953 29.8) (width 0.2) (layer "F.Cu") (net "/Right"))
 (segment (start 42.2465 33.356) (end 43.159 32.4435) (width 0.2) (layer "F.Cu") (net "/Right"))
 (segment (start 38.563 31.616) (end 40.303 33.356) (width 0.2) (layer "F.Cu") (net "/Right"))
 (segment (start 40.303 33.356) (end 42.2465 33.356) (width 0.2) (layer "F.Cu") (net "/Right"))
 (segment (start 38.563 30.016) (end 40.073 30.016) (width 0.2) (layer "F.Cu") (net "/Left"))
 (segment (start 41.635 31.578) (end 45.953 27.26) (width 0.2) (layer "F.Cu") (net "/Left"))
 (segment (start 40.073 30.016) (end 41.635 31.578) (width 0.2) (layer "F.Cu") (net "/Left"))
 (segment (start 41.635 32.4435) (end 41.635 31.578) (width 0.2) (layer "F.Cu") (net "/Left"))
 (segment (start 38.587 27.6145) (end 37.463 28.7385) (width 0.2) (layer "F.Cu") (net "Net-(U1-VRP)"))
 (segment (start 37.463 28.7385) (end 37.463 29.316) (width 0.2) (layer "F.Cu") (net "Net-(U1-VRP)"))
 (segment (start 37.063 27.6145) (end 37.063 29.316) (width 0.2) (layer "F.Cu") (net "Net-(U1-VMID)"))
 (segment (start 36.663 28.716) (end 36.663 29.316) (width 0.2) (layer "F.Cu") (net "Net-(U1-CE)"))
 (segment (start 35.6115 27.6645) (end 36.663 28.716) (width 0.2) (layer "F.Cu") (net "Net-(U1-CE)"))
 (segment (start 35.539 27.6645) (end 35.6115 27.6645) (width 0.2) (layer "F.Cu") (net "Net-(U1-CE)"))
 (segment (start 43.159 40.238) (end 43.159 34.2685) (width 0.2) (layer "F.Cu") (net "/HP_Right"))
 (segment (start 41.453 41.944) (end 43.159 40.238) (width 0.2) (layer "F.Cu") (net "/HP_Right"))
 (segment (start 41.635 34.2685) (end 41.635 37.762) (width 0.2) (layer "F.Cu") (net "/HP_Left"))
 (segment (start 41.635 37.762) (end 37.453 41.944) (width 0.2) (layer "F.Cu") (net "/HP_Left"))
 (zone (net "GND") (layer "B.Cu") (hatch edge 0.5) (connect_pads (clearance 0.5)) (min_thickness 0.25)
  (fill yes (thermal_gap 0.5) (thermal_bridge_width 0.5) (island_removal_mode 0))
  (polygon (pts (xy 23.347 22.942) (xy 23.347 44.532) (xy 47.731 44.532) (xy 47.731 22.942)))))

